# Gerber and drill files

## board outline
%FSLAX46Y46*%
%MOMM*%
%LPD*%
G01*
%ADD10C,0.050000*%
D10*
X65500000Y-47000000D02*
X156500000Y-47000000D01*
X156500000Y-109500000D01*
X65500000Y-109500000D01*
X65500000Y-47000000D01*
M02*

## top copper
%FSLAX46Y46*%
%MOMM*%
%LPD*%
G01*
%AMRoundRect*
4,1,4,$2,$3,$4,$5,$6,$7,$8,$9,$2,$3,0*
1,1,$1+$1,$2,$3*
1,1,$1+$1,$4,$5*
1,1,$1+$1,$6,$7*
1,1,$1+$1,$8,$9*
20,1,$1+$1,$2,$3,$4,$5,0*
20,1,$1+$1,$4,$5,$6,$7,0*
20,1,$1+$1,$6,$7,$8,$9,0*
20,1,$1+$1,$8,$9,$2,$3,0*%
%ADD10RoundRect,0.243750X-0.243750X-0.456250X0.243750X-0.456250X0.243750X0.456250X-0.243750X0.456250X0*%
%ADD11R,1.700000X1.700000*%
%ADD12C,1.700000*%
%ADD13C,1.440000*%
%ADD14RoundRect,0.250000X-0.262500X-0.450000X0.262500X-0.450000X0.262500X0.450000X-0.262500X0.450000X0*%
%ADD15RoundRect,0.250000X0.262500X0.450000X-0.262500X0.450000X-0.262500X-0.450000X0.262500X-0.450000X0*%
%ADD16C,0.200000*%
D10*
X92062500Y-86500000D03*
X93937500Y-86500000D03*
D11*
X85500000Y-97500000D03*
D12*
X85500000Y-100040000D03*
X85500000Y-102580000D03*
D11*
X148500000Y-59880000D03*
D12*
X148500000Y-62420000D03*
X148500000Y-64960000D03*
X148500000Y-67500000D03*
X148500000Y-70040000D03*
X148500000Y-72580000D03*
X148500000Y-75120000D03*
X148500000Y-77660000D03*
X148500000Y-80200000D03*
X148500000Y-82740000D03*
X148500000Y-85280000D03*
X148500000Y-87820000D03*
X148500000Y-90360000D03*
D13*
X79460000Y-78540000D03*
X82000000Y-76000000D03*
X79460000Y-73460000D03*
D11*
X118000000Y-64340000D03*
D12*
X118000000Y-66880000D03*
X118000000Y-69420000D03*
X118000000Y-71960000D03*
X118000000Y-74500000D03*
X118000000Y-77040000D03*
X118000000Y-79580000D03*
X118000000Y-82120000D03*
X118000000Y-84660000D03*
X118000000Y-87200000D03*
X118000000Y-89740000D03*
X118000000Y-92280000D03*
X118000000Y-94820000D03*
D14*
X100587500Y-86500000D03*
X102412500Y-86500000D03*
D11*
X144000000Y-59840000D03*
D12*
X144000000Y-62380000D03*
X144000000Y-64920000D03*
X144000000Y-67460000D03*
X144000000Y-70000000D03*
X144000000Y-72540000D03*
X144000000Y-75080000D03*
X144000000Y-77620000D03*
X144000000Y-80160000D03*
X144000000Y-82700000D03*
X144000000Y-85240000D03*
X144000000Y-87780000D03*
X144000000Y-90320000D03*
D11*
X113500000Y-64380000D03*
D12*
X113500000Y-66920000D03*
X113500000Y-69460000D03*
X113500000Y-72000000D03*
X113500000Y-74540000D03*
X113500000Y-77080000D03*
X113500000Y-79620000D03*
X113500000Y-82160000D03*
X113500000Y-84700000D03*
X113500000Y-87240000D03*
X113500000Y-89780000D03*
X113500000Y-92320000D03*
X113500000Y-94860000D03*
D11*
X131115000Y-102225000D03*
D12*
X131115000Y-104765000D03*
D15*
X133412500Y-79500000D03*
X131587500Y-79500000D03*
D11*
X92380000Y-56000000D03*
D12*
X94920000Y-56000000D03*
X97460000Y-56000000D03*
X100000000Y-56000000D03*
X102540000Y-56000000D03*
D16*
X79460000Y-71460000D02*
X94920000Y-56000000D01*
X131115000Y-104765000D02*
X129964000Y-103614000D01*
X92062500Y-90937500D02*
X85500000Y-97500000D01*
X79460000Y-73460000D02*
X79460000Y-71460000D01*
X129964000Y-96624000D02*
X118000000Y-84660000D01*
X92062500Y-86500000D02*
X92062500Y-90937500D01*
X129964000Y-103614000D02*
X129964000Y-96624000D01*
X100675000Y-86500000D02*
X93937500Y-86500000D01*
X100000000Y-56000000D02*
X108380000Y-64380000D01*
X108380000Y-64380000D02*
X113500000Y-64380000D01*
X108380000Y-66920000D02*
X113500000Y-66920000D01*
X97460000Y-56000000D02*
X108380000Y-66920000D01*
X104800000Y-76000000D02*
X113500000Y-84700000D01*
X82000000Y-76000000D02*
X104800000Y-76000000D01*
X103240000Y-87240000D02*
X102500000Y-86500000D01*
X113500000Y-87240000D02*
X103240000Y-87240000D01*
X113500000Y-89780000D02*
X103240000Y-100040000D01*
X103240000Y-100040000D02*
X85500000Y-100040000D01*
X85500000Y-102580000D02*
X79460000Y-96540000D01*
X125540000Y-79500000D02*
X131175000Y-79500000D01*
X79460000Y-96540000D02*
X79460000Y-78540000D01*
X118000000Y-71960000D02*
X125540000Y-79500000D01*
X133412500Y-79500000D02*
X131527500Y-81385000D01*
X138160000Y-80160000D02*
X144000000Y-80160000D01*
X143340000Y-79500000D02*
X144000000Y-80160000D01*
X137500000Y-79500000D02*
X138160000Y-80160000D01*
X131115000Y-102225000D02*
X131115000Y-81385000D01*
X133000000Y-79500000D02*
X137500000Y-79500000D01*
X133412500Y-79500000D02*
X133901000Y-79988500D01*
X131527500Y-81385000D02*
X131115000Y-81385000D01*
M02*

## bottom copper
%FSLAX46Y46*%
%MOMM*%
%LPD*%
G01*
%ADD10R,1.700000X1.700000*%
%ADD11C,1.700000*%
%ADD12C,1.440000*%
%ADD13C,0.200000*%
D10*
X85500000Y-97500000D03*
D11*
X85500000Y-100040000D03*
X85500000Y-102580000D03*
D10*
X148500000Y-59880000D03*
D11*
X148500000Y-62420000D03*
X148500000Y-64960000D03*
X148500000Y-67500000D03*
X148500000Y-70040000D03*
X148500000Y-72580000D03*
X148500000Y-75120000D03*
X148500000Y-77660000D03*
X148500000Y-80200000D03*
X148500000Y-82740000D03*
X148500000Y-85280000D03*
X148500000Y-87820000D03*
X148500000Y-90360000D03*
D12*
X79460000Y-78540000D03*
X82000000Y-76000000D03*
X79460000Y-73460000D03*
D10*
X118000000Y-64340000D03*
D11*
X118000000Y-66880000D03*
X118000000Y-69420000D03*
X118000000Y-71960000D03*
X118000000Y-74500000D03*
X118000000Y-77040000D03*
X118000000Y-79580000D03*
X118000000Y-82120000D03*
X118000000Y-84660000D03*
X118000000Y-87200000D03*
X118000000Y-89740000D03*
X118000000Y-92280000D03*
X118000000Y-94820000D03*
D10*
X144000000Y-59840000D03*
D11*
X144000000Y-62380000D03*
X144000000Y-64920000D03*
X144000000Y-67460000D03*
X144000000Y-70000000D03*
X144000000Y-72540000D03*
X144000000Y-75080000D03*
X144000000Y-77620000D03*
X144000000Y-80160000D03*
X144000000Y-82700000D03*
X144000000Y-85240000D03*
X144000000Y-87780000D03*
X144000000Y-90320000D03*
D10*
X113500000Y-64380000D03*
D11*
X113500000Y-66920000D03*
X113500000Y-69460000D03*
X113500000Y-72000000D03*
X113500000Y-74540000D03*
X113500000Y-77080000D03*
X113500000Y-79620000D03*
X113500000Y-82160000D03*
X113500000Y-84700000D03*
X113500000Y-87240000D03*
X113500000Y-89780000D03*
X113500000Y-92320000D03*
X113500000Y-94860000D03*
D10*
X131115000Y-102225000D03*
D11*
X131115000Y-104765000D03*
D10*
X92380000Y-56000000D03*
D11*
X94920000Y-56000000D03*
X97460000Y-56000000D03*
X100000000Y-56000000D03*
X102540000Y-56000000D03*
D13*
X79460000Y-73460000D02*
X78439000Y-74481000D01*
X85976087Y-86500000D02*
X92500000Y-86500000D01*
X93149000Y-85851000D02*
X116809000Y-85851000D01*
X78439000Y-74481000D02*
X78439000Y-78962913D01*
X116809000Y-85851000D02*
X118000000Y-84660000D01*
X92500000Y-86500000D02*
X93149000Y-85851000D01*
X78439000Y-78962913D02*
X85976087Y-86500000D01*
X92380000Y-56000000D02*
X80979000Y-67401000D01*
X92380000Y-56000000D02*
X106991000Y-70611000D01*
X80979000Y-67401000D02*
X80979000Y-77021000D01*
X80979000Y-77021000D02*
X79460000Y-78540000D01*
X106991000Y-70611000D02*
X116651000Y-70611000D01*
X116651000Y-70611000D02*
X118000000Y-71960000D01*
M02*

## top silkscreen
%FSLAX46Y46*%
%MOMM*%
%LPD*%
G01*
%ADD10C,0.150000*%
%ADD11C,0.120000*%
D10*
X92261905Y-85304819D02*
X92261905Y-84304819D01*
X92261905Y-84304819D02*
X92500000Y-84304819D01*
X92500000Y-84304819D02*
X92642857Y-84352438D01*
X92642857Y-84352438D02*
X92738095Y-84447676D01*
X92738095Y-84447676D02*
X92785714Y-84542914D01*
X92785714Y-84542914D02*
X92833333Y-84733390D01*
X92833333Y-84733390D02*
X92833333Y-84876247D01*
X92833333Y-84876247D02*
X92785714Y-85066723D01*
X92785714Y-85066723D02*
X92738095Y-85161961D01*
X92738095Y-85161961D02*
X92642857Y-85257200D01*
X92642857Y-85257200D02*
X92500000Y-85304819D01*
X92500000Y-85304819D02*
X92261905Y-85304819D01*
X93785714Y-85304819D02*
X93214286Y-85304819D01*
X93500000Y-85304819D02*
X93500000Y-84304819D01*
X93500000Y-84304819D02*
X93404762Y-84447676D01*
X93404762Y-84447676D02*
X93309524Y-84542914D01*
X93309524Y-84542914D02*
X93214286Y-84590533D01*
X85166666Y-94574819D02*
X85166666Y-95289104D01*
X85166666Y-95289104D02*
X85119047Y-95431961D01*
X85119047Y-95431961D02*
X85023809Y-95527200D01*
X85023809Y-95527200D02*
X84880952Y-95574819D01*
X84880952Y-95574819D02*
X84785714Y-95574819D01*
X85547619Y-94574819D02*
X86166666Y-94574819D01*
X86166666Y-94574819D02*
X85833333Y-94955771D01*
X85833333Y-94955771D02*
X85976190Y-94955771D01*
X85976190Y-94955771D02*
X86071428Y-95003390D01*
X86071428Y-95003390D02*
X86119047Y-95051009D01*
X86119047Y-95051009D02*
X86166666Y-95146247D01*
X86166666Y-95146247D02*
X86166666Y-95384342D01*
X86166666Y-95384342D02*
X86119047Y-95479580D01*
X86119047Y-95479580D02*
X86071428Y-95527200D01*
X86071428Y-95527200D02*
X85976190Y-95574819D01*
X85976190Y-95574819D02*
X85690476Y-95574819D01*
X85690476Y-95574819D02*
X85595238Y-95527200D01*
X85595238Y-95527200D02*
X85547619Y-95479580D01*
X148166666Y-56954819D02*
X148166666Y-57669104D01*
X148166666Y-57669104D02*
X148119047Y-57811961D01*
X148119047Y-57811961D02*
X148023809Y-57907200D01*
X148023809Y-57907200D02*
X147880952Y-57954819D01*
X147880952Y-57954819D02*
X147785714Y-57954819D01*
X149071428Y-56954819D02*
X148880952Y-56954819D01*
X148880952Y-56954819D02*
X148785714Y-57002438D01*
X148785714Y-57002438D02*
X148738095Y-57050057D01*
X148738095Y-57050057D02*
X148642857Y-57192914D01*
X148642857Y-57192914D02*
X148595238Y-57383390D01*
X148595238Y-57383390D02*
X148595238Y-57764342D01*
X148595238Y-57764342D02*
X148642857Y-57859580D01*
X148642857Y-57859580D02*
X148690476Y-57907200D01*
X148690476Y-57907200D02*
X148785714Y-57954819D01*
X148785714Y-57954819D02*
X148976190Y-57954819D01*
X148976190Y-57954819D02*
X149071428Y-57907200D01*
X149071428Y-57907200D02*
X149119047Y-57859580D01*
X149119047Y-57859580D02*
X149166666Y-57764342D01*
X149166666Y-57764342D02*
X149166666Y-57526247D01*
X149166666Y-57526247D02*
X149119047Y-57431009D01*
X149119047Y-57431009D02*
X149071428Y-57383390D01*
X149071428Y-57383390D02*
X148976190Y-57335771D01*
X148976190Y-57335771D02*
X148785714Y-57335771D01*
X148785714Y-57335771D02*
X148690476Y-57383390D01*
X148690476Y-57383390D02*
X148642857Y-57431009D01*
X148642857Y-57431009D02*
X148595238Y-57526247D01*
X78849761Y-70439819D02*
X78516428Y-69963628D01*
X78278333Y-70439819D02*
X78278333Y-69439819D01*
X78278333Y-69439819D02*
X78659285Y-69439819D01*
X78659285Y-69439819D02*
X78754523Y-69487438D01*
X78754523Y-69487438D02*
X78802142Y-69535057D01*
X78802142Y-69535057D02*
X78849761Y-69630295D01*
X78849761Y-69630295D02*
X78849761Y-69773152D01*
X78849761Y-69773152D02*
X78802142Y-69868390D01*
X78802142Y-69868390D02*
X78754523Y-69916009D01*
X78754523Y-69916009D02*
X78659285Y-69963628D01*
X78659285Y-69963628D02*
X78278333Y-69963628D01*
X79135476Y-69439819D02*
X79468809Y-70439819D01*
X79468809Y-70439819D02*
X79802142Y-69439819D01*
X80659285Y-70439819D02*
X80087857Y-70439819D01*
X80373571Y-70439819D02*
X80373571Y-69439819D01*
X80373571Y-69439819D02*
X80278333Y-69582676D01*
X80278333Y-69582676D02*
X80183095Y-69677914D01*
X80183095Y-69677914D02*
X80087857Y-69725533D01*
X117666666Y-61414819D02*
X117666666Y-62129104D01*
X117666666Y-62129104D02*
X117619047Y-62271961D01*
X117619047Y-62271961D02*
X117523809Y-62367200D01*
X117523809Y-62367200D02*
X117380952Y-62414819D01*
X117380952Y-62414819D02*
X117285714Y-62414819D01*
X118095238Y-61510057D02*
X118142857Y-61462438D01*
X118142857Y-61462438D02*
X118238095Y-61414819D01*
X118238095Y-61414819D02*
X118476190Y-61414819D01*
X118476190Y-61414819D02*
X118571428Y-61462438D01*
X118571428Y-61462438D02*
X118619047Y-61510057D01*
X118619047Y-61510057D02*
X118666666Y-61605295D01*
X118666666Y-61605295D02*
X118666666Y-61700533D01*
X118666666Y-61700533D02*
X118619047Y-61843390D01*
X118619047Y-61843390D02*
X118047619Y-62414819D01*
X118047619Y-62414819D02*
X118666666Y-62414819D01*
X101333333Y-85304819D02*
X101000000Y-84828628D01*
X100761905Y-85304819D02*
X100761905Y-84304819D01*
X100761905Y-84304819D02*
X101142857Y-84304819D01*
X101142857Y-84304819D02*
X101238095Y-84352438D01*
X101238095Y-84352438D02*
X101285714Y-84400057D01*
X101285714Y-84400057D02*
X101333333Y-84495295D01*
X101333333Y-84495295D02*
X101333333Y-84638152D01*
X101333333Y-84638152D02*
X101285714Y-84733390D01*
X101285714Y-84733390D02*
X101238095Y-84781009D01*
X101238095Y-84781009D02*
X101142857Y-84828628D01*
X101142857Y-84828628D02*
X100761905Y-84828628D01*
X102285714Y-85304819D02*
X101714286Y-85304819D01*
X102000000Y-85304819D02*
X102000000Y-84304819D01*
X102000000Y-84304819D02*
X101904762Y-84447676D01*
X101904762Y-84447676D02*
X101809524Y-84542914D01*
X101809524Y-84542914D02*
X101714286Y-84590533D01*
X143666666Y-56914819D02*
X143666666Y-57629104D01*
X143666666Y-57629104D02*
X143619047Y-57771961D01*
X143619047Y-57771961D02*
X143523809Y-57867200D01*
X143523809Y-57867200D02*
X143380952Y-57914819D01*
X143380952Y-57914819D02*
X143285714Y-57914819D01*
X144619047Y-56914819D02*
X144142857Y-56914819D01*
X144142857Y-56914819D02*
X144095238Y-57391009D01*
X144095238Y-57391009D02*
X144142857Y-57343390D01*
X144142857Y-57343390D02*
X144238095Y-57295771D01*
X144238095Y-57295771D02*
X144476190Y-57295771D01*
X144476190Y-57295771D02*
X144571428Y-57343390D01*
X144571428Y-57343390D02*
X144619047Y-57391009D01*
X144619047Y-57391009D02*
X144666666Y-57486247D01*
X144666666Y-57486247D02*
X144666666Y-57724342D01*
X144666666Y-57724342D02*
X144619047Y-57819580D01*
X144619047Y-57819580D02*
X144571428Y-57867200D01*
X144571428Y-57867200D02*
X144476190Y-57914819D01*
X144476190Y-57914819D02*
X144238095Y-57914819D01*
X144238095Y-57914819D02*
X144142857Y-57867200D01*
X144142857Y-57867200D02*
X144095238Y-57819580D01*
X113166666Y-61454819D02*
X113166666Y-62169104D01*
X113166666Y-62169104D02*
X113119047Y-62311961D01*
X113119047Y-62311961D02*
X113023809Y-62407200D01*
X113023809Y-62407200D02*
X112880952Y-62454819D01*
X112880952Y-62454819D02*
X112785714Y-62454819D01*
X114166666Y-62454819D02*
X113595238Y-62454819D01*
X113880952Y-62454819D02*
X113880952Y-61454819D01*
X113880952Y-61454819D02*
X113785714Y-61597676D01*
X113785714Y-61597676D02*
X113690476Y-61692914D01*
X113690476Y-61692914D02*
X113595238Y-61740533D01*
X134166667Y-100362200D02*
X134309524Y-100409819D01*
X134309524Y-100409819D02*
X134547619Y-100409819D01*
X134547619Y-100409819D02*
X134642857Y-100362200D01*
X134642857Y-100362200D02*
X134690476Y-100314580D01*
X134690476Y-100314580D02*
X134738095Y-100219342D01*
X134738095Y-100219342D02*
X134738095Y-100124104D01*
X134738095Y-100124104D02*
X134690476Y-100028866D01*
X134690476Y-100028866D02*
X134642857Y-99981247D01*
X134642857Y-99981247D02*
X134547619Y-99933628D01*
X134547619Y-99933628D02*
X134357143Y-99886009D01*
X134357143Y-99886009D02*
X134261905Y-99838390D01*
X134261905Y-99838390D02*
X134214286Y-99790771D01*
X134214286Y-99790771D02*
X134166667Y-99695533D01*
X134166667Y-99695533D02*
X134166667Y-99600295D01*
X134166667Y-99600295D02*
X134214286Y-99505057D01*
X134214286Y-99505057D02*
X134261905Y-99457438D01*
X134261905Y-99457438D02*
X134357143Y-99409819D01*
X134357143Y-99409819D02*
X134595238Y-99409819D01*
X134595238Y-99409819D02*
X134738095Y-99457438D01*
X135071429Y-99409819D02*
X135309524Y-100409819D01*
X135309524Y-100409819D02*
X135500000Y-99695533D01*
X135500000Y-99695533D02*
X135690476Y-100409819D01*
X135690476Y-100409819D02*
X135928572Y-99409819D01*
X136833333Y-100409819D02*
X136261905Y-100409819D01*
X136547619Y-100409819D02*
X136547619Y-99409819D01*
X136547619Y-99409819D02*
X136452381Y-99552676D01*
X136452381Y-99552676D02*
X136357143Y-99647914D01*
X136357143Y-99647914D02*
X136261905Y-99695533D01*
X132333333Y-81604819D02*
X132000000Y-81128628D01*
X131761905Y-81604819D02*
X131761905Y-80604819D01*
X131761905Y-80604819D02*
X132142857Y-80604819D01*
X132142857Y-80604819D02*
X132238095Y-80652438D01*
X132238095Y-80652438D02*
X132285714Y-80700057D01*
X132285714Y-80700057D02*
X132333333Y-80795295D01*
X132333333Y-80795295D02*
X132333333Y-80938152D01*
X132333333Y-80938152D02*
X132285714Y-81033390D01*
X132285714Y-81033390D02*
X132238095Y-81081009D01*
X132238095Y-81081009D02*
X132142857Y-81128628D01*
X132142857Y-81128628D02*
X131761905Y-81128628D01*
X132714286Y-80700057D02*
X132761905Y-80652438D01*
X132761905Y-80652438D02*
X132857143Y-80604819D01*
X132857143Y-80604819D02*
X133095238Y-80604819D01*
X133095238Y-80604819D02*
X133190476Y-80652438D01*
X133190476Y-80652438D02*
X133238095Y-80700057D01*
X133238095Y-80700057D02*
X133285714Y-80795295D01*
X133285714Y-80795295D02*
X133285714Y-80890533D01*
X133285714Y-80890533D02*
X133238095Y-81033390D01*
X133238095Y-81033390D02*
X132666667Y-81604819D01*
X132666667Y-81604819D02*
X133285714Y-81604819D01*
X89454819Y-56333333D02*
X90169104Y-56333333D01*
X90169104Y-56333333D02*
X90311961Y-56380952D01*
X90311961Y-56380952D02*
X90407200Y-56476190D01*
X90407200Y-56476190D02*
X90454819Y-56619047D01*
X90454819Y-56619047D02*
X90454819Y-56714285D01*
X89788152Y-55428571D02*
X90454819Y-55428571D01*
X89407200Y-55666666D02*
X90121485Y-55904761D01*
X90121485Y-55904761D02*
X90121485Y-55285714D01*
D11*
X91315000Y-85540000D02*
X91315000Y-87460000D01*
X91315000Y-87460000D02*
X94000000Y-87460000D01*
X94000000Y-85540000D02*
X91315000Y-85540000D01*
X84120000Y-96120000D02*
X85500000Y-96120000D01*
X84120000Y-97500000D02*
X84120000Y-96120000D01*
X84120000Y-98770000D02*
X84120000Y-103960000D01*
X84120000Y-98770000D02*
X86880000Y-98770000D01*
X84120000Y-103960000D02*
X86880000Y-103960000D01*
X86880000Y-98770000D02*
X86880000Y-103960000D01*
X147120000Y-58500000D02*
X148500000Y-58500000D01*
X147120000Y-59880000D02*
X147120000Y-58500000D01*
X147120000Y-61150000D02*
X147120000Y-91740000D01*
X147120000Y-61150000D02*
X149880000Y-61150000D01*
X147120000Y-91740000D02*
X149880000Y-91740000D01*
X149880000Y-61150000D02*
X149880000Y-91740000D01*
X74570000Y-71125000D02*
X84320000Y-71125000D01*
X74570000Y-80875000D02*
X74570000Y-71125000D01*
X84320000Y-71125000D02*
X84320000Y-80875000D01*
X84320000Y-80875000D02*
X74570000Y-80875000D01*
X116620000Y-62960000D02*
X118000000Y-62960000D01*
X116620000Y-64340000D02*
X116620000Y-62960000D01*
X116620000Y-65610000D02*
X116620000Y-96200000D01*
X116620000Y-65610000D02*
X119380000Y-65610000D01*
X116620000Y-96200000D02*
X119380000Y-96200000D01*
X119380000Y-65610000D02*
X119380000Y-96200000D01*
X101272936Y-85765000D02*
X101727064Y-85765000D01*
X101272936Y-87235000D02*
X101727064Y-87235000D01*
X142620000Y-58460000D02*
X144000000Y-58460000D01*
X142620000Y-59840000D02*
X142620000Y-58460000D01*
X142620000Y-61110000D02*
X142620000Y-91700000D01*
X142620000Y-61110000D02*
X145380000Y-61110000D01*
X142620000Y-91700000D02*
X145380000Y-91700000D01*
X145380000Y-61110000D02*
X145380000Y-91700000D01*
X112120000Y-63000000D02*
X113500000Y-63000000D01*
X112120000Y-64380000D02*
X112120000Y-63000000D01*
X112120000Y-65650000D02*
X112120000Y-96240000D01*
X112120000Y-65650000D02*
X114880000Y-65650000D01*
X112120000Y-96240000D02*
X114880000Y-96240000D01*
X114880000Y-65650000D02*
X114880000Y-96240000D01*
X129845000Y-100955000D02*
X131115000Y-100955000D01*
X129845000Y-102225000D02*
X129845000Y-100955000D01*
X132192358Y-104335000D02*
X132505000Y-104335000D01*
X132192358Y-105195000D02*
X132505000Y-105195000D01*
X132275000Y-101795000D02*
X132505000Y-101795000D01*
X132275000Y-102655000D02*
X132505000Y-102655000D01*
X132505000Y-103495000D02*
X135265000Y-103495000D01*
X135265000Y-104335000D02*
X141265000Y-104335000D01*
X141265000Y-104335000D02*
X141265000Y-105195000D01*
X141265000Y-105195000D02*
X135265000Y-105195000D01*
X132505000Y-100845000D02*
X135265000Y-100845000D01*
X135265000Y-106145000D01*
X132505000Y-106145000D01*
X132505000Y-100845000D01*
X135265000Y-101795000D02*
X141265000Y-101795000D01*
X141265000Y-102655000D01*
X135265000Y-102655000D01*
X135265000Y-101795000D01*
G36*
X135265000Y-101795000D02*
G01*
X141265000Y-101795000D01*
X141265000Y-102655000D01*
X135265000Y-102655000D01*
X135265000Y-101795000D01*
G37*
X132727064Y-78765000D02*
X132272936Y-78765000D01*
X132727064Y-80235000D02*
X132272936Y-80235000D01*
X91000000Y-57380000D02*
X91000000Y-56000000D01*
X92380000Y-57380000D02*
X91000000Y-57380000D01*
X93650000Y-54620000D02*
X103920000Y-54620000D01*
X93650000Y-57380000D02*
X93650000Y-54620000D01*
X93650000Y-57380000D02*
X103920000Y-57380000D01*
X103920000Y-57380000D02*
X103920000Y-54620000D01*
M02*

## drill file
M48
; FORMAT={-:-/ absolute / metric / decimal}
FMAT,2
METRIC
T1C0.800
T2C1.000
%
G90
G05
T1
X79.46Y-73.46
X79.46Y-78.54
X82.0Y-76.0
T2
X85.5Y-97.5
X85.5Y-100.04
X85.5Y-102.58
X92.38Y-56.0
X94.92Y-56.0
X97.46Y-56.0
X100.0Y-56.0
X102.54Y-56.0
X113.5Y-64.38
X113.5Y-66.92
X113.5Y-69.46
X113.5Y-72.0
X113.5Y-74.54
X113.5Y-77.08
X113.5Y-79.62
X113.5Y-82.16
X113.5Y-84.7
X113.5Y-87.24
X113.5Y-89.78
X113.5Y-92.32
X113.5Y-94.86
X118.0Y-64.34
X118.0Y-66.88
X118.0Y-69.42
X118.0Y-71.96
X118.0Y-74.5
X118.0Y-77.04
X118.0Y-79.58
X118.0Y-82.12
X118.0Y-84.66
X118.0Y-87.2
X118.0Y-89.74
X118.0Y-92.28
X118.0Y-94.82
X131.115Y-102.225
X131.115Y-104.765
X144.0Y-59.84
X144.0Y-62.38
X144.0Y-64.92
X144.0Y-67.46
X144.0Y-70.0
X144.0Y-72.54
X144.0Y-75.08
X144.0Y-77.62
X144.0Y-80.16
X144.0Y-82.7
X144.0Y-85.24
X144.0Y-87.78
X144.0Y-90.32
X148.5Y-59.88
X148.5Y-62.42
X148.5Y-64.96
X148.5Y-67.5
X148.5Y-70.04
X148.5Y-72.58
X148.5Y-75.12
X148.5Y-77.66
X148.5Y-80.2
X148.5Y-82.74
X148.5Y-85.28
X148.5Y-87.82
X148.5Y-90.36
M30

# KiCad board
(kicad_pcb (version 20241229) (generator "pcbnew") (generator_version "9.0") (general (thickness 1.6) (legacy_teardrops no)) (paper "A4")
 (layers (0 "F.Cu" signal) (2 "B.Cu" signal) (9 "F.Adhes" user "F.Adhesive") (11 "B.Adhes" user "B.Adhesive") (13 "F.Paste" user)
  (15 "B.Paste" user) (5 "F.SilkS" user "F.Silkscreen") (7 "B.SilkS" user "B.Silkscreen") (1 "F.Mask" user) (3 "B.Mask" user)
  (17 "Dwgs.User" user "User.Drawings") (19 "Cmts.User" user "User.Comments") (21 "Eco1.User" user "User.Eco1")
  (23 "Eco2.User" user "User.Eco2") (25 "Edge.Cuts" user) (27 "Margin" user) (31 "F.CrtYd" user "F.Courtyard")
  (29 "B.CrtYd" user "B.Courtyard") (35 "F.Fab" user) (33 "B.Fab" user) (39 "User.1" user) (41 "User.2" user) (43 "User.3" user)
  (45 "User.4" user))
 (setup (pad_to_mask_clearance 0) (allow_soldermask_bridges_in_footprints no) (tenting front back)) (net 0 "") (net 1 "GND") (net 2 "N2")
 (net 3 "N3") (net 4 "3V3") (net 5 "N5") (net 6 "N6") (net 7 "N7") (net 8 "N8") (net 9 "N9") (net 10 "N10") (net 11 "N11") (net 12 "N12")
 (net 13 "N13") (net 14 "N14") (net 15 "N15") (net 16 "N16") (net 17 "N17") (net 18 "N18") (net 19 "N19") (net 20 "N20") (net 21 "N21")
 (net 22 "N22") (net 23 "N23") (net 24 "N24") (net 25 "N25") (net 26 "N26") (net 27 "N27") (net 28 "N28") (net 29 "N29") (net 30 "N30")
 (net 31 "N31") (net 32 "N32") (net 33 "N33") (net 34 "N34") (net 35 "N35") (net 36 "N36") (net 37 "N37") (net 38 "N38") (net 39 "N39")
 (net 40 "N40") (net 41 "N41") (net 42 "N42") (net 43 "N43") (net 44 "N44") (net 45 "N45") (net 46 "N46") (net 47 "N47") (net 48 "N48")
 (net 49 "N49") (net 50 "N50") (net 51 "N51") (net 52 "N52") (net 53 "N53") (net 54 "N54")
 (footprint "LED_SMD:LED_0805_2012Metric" (layer "F.Cu") (at 93 86.5)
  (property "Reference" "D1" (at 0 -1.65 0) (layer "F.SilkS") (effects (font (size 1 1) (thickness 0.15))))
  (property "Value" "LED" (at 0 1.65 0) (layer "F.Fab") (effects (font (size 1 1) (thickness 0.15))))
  (fp_line (start -1.685 -0.96) (end -1.685 0.96) (stroke (width 0.12) (type solid)) (layer "F.SilkS"))
  (fp_line (start -1.685 0.96) (end 1 0.96) (stroke (width 0.12) (type solid)) (layer "F.SilkS"))
  (fp_line (start 1 -0.96) (end -1.685 -0.96) (stroke (width 0.12) (type solid)) (layer "F.SilkS"))
  (pad "1" smd roundrect (at -0.9375 0) (size 0.975 1.4) (layers "F.Cu" "F.Mask" "F.Paste") (roundrect_rratio 0.25) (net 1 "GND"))
  (pad "2" smd roundrect (at 0.9375 0) (size 0.975 1.4) (layers "F.Cu" "F.Mask" "F.Paste") (roundrect_rratio 0.25) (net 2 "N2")))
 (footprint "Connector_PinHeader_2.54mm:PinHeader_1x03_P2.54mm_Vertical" (layer "F.Cu") (at 85.5 97.5)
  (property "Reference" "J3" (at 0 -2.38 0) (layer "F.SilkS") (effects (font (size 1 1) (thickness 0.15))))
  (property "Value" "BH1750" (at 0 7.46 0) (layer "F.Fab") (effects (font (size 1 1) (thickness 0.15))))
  (fp_line (start -1.38 -1.38) (end 0 -1.38) (stroke (width 0.12) (type solid)) (layer "F.SilkS"))
  (fp_line (start -1.38 0) (end -1.38 -1.38) (stroke (width 0.12) (type solid)) (layer "F.SilkS"))
  (fp_line (start -1.38 1.27) (end -1.38 6.46) (stroke (width 0.12) (type solid)) (layer "F.SilkS"))
  (fp_line (start -1.38 1.27) (end 1.38 1.27) (stroke (width 0.12) (type solid)) (layer "F.SilkS"))
  (fp_line (start -1.38 6.46) (end 1.38 6.46) (stroke (width 0.12) (type solid)) (layer "F.SilkS"))
  (fp_line (start 1.38 1.27) (end 1.38 6.46) (stroke (width 0.12) (type solid)) (layer "F.SilkS"))
  (pad "1" thru_hole rect (at 0 0) (size 1.7 1.7) (drill 1) (layers "*.Cu" "*.Mask") (remove_unused_layers no) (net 1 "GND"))
  (pad "2" thru_hole circle (at 0 2.54) (size 1.7 1.7) (drill 1) (layers "*.Cu" "*.Mask") (remove_unused_layers no) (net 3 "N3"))
  (pad "3" thru_hole circle (at 0 5.08) (size 1.7 1.7) (drill 1) (layers "*.Cu" "*.Mask") (remove_unused_layers no) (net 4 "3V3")))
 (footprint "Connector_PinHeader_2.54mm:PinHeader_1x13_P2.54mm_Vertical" (layer "F.Cu") (at 148.5 59.88)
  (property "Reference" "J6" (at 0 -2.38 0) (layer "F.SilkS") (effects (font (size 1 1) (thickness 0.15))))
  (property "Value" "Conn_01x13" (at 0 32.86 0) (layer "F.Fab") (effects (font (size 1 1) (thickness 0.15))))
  (fp_line (start -1.38 -1.38) (end 0 -1.38) (stroke (width 0.12) (type solid)) (layer "F.SilkS"))
  (fp_line (start -1.38 0) (end -1.38 -1.38) (stroke (width 0.12) (type solid)) (layer "F.SilkS"))
  (fp_line (start -1.38 1.27) (end -1.38 31.86) (stroke (width 0.12) (type solid)) (layer "F.SilkS"))
  (fp_line (start -1.38 1.27) (end 1.38 1.27) (stroke (width 0.12) (type solid)) (layer "F.SilkS"))
  (fp_line (start -1.38 31.86) (end 1.38 31.86) (stroke (width 0.12) (type solid)) (layer "F.SilkS"))
  (fp_line (start 1.38 1.27) (end 1.38 31.86) (stroke (width 0.12) (type solid)) (layer "F.SilkS"))
  (pad "1" thru_hole rect (at 0 0) (size 1.7 1.7) (drill 1) (layers "*.Cu" "*.Mask") (remove_unused_layers no) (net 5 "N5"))
  (pad "2" thru_hole circle (at 0 2.54) (size 1.7 1.7) (drill 1) (layers "*.Cu" "*.Mask") (remove_unused_layers no) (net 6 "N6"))
  (pad "3" thru_hole circle (at 0 5.08) (size 1.7 1.7) (drill 1) (layers "*.Cu" "*.Mask") (remove_unused_layers no) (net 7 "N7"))
  (pad "4" thru_hole circle (at 0 7.62) (size 1.7 1.7) (drill 1) (layers "*.Cu" "*.Mask") (remove_unused_layers no) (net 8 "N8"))
  (pad "5" thru_hole circle (at 0 10.16) (size 1.7 1.7) (drill 1) (layers "*.Cu" "*.Mask") (remove_unused_layers no) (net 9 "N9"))
  (pad "6" thru_hole circle (at 0 12.7) (size 1.7 1.7) (drill 1) (layers "*.Cu" "*.Mask") (remove_unused_layers no) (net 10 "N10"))
  (pad "7" thru_hole circle (at 0 15.24) (size 1.7 1.7) (drill 1) (layers "*.Cu" "*.Mask") (remove_unused_layers no) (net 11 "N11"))
  (pad "8" thru_hole circle (at 0 17.78) (size 1.7 1.7) (drill 1) (layers "*.Cu" "*.Mask") (remove_unused_layers no) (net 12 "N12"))
  (pad "9" thru_hole circle (at 0 20.32) (size 1.7 1.7) (drill 1) (layers "*.Cu" "*.Mask") (remove_unused_layers no) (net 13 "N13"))
  (pad "10" thru_hole circle (at 0 22.86) (size 1.7 1.7) (drill 1) (layers "*.Cu" "*.Mask") (remove_unused_layers no) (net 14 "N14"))
  (pad "11" thru_hole circle (at 0 25.4) (size 1.7 1.7) (drill 1) (layers "*.Cu" "*.Mask") (remove_unused_layers no) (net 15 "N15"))
  (pad "12" thru_hole circle (at 0 27.94) (size 1.7 1.7) (drill 1) (layers "*.Cu" "*.Mask") (remove_unused_layers no) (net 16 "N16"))
  (pad "13" thru_hole circle (at 0 30.48) (size 1.7 1.7) (drill 1) (layers "*.Cu" "*.Mask") (remove_unused_layers no) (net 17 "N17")))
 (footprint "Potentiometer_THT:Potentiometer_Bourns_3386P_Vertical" (layer "F.Cu") (at 79.46 78.54)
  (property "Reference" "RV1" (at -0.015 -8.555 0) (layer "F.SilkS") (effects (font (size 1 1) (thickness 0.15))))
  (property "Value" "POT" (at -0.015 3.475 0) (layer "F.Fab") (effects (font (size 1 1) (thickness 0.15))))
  (fp_line (start -4.89 -7.415) (end 4.86 -7.415) (stroke (width 0.12) (type solid)) (layer "F.SilkS"))
  (fp_line (start -4.89 2.335) (end -4.89 -7.415) (stroke (width 0.12) (type solid)) (layer "F.SilkS"))
  (fp_line (start 4.86 -7.415) (end 4.86 2.335) (stroke (width 0.12) (type solid)) (layer "F.SilkS"))
  (fp_line (start 4.86 2.335) (end -4.89 2.335) (stroke (width 0.12) (type solid)) (layer "F.SilkS"))
  (pad "1" thru_hole circle (at 0 0) (size 1.44 1.44) (drill 0.8) (layers "*.Cu" "*.Mask") (remove_unused_layers no) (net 4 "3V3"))
  (pad "2" thru_hole circle (at 2.54 -2.54) (size 1.44 1.44) (drill 0.8) (layers "*.Cu" "*.Mask") (remove_unused_layers no) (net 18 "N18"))
  (pad "3" thru_hole circle (at 0 -5.08) (size 1.44 1.44) (drill 0.8) (layers "*.Cu" "*.Mask") (remove_unused_layers no) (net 1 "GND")))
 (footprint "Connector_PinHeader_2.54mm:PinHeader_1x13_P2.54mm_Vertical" (layer "F.Cu") (at 118 64.34)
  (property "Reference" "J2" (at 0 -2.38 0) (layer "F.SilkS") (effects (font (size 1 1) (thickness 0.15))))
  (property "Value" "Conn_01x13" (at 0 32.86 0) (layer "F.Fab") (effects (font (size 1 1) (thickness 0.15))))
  (fp_line (start -1.38 -1.38) (end 0 -1.38) (stroke (width 0.12) (type solid)) (layer "F.SilkS"))
  (fp_line (start -1.38 0) (end -1.38 -1.38) (stroke (width 0.12) (type solid)) (layer "F.SilkS"))
  (fp_line (start -1.38 1.27) (end -1.38 31.86) (stroke (width 0.12) (type solid)) (layer "F.SilkS"))
  (fp_line (start -1.38 1.27) (end 1.38 1.27) (stroke (width 0.12) (type solid)) (layer "F.SilkS"))
  (fp_line (start -1.38 31.86) (end 1.38 31.86) (stroke (width 0.12) (type solid)) (layer "F.SilkS"))
  (fp_line (start 1.38 1.27) (end 1.38 31.86) (stroke (width 0.12) (type solid)) (layer "F.SilkS"))
  (pad "1" thru_hole rect (at 0 0) (size 1.7 1.7) (drill 1) (layers "*.Cu" "*.Mask") (remove_unused_layers no) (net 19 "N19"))
  (pad "2" thru_hole circle (at 0 2.54) (size 1.7 1.7) (drill 1) (layers "*.Cu" "*.Mask") (remove_unused_layers no) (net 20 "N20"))
  (pad "3" thru_hole circle (at 0 5.08) (size 1.7 1.7) (drill 1) (layers "*.Cu" "*.Mask") (remove_unused_layers no) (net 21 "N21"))
  (pad "4" thru_hole circle (at 0 7.62) (size 1.7 1.7) (drill 1) (layers "*.Cu" "*.Mask") (remove_unused_layers no) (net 4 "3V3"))
  (pad "5" thru_hole circle (at 0 10.16) (size 1.7 1.7) (drill 1) (layers "*.Cu" "*.Mask") (remove_unused_layers no) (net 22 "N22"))
  (pad "6" thru_hole circle (at 0 12.7) (size 1.7 1.7) (drill 1) (layers "*.Cu" "*.Mask") (remove_unused_layers no) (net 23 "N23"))
  (pad "7" thru_hole circle (at 0 15.24) (size 1.7 1.7) (drill 1) (layers "*.Cu" "*.Mask") (remove_unused_layers no) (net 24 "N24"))
  (pad "8" thru_hole circle (at 0 17.78) (size 1.7 1.7) (drill 1) (layers "*.Cu" "*.Mask") (remove_unused_layers no) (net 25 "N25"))
  (pad "9" thru_hole circle (at 0 20.32) (size 1.7 1.7) (drill 1) (layers "*.Cu" "*.Mask") (remove_unused_layers no) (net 1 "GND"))
  (pad "10" thru_hole circle (at 0 22.86) (size 1.7 1.7) (drill 1) (layers "*.Cu" "*.Mask") (remove_unused_layers no) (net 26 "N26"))
  (pad "11" thru_hole circle (at 0 25.4) (size 1.7 1.7) (drill 1) (layers "*.Cu" "*.Mask") (remove_unused_layers no) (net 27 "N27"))
  (pad "12" thru_hole circle (at 0 27.94) (size 1.7 1.7) (drill 1) (layers "*.Cu" "*.Mask") (remove_unused_layers no) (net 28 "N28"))
  (pad "13" thru_hole circle (at 0 30.48) (size 1.7 1.7) (drill 1) (layers "*.Cu" "*.Mask") (remove_unused_layers no) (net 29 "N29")))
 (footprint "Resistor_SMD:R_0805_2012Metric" (layer "F.Cu") (at 101.5 86.5)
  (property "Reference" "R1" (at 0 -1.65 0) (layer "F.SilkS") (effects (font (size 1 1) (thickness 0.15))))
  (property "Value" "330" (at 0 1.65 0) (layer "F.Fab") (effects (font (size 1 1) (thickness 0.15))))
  (fp_line (start -0.227064 -0.735) (end 0.227064 -0.735) (stroke (width 0.12) (type solid)) (layer "F.SilkS"))
  (fp_line (start -0.227064 0.735) (end 0.227064 0.735) (stroke (width 0.12) (type solid)) (layer "F.SilkS"))
  (pad "1" smd roundrect (at -0.9125 0) (size 1.025 1.4) (layers "F.Cu" "F.Mask" "F.Paste") (roundrect_rratio 0.243902) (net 2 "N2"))
  (pad "2" smd roundrect (at 0.9125 0) (size 1.025 1.4) (layers "F.Cu" "F.Mask" "F.Paste") (roundrect_rratio 0.243902) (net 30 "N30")))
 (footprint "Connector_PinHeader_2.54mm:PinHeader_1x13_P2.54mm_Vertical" (layer "F.Cu") (at 144 59.84)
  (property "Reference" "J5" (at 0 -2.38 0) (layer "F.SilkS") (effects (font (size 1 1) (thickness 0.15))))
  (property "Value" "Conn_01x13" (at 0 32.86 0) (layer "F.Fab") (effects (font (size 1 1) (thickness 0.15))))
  (fp_line (start -1.38 -1.38) (end 0 -1.38) (stroke (width 0.12) (type solid)) (layer "F.SilkS"))
  (fp_line (start -1.38 0) (end -1.38 -1.38) (stroke (width 0.12) (type solid)) (layer "F.SilkS"))
  (fp_line (start -1.38 1.27) (end -1.38 31.86) (stroke (width 0.12) (type solid)) (layer "F.SilkS"))
  (fp_line (start -1.38 1.27) (end 1.38 1.27) (stroke (width 0.12) (type solid)) (layer "F.SilkS"))
  (fp_line (start -1.38 31.86) (end 1.38 31.86) (stroke (width 0.12) (type solid)) (layer "F.SilkS"))
  (fp_line (start 1.38 1.27) (end 1.38 31.86) (stroke (width 0.12) (type solid)) (layer "F.SilkS"))
  (pad "1" thru_hole rect (at 0 0) (size 1.7 1.7) (drill 1) (layers "*.Cu" "*.Mask") (remove_unused_layers no) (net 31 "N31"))
  (pad "2" thru_hole circle (at 0 2.54) (size 1.7 1.7) (drill 1) (layers "*.Cu" "*.Mask") (remove_unused_layers no) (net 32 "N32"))
  (pad "3" thru_hole circle (at 0 5.08) (size 1.7 1.7) (drill 1) (layers "*.Cu" "*.Mask") (remove_unused_layers no) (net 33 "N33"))
  (pad "4" thru_hole circle (at 0 7.62) (size 1.7 1.7) (drill 1) (layers "*.Cu" "*.Mask") (remove_unused_layers no) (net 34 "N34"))
  (pad "5" thru_hole circle (at 0 10.16) (size 1.7 1.7) (drill 1) (layers "*.Cu" "*.Mask") (remove_unused_layers no) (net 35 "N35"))
  (pad "6" thru_hole circle (at 0 12.7) (size 1.7 1.7) (drill 1) (layers "*.Cu" "*.Mask") (remove_unused_layers no) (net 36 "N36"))
  (pad "7" thru_hole circle (at 0 15.24) (size 1.7 1.7) (drill 1) (layers "*.Cu" "*.Mask") (remove_unused_layers no) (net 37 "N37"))
  (pad "8" thru_hole circle (at 0 17.78) (size 1.7 1.7) (drill 1) (layers "*.Cu" "*.Mask") (remove_unused_layers no) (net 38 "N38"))
  (pad "9" thru_hole circle (at 0 20.32) (size 1.7 1.7) (drill 1) (layers "*.Cu" "*.Mask") (remove_unused_layers no) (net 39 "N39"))
  (pad "10" thru_hole circle (at 0 22.86) (size 1.7 1.7) (drill 1) (layers "*.Cu" "*.Mask") (remove_unused_layers no) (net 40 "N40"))
  (pad "11" thru_hole circle (at 0 25.4) (size 1.7 1.7) (drill 1) (layers "*.Cu" "*.Mask") (remove_unused_layers no) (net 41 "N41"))
  (pad "12" thru_hole circle (at 0 27.94) (size 1.7 1.7) (drill 1) (layers "*.Cu" "*.Mask") (remove_unused_layers no) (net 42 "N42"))
  (pad "13" thru_hole circle (at 0 30.48) (size 1.7 1.7) (drill 1) (layers "*.Cu" "*.Mask") (remove_unused_layers no) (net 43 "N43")))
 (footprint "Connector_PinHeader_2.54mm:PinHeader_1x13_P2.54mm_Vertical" (layer "F.Cu") (at 113.5 64.38)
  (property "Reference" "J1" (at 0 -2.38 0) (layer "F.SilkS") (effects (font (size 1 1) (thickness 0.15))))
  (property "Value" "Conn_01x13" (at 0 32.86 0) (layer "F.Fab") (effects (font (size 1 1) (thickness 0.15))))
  (fp_line (start -1.38 -1.38) (end 0 -1.38) (stroke (width 0.12) (type solid)) (layer "F.SilkS"))
  (fp_line (start -1.38 0) (end -1.38 -1.38) (stroke (width 0.12) (type solid)) (layer "F.SilkS"))
  (fp_line (start -1.38 1.27) (end -1.38 31.86) (stroke (width 0.12) (type solid)) (layer "F.SilkS"))
  (fp_line (start -1.38 1.27) (end 1.38 1.27) (stroke (width 0.12) (type solid)) (layer "F.SilkS"))
  (fp_line (start -1.38 31.86) (end 1.38 31.86) (stroke (width 0.12) (type solid)) (layer "F.SilkS"))
  (fp_line (start 1.38 1.27) (end 1.38 31.86) (stroke (width 0.12) (type solid)) (layer "F.SilkS"))
  (pad "1" thru_hole rect (at 0 0) (size 1.7 1.7) (drill 1) (layers "*.Cu" "*.Mask") (remove_unused_layers no) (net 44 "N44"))
  (pad "2" thru_hole circle (at 0 2.54) (size 1.7 1.7) (drill 1) (layers "*.Cu" "*.Mask") (remove_unused_layers no) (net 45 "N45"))
  (pad "3" thru_hole circle (at 0 5.08) (size 1.7 1.7) (drill 1) (layers "*.Cu" "*.Mask") (remove_unused_layers no) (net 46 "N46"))
  (pad "4" thru_hole circle (at 0 7.62) (size 1.7 1.7) (drill 1) (layers "*.Cu" "*.Mask") (remove_unused_layers no) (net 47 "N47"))
  (pad "5" thru_hole circle (at 0 10.16) (size 1.7 1.7) (drill 1) (layers "*.Cu" "*.Mask") (remove_unused_layers no) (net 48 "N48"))
  (pad "6" thru_hole circle (at 0 12.7) (size 1.7 1.7) (drill 1) (layers "*.Cu" "*.Mask") (remove_unused_layers no) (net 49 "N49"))
  (pad "7" thru_hole circle (at 0 15.24) (size 1.7 1.7) (drill 1) (layers "*.Cu" "*.Mask") (remove_unused_layers no) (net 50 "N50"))
  (pad "8" thru_hole circle (at 0 17.78) (size 1.7 1.7) (drill 1) (layers "*.Cu" "*.Mask") (remove_unused_layers no) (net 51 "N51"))
  (pad "9" thru_hole circle (at 0 20.32) (size 1.7 1.7) (drill 1) (layers "*.Cu" "*.Mask") (remove_unused_layers no) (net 18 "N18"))
  (pad "10" thru_hole circle (at 0 22.86) (size 1.7 1.7) (drill 1) (layers "*.Cu" "*.Mask") (remove_unused_layers no) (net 30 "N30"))
  (pad "11" thru_hole circle (at 0 25.4) (size 1.7 1.7) (drill 1) (layers "*.Cu" "*.Mask") (remove_unused_layers no) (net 3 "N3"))
  (pad "12" thru_hole circle (at 0 27.94) (size 1.7 1.7) (drill 1) (layers "*.Cu" "*.Mask") (remove_unused_layers no) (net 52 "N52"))
  (pad "13" thru_hole circle (at 0 30.48) (size 1.7 1.7) (drill 1) (layers "*.Cu" "*.Mask") (remove_unused_layers no) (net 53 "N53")))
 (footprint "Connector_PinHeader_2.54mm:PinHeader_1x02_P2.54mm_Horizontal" (layer "F.Cu") (at 131.115 102.225)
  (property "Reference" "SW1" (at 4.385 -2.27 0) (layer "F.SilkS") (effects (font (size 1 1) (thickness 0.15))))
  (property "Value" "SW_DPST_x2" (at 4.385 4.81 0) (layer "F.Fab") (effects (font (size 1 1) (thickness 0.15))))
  (fp_line (start -1.27 -1.27) (end 0 -1.27) (stroke (width 0.12) (type solid)) (layer "F.SilkS"))
  (fp_line (start -1.27 0) (end -1.27 -1.27) (stroke (width 0.12) (type solid)) (layer "F.SilkS"))
  (fp_line (start 1.077358 2.11) (end 1.39 2.11) (stroke (width 0.12) (type solid)) (layer "F.SilkS"))
  (fp_line (start 1.077358 2.97) (end 1.39 2.97) (stroke (width 0.12) (type solid)) (layer "F.SilkS"))
  (fp_line (start 1.16 -0.43) (end 1.39 -0.43) (stroke (width 0.12) (type solid)) (layer "F.SilkS"))
  (fp_line (start 1.16 0.43) (end 1.39 0.43) (stroke (width 0.12) (type solid)) (layer "F.SilkS"))
  (fp_line (start 1.39 1.27) (end 4.15 1.27) (stroke (width 0.12) (type solid)) (layer "F.SilkS"))
  (fp_line (start 4.15 2.11) (end 10.15 2.11) (stroke (width 0.12) (type solid)) (layer "F.SilkS"))
  (fp_line (start 10.15 2.11) (end 10.15 2.97) (stroke (width 0.12) (type solid)) (layer "F.SilkS"))
  (fp_line (start 10.15 2.97) (end 4.15 2.97) (stroke (width 0.12) (type solid)) (layer "F.SilkS"))
  (fp_rect (start 1.39 -1.38) (end 4.15 3.92) (stroke (width 0.12) (type solid)) (fill no) (layer "F.SilkS"))
  (fp_rect (start 4.15 -0.43) (end 10.15 0.43) (stroke (width 0.12) (type solid)) (fill yes) (layer "F.SilkS"))
  (pad "1" thru_hole rect (at 0 0) (size 1.7 1.7) (drill 1) (layers "*.Cu" "*.Mask") (remove_unused_layers no) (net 39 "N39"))
  (pad "2" thru_hole circle (at 0 2.54) (size 1.7 1.7) (drill 1) (layers "*.Cu" "*.Mask") (remove_unused_layers no) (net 1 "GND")))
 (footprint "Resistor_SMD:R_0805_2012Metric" (layer "F.Cu") (at 132.5 79.5 180)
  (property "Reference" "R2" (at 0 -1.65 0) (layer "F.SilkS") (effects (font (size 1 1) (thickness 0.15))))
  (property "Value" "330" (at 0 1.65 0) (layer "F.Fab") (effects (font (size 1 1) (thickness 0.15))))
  (fp_line (start -0.227064 0.735) (end 0.227064 0.735) (stroke (width 0.12) (type solid)) (layer "F.SilkS"))
  (fp_line (start -0.227064 -0.735) (end 0.227064 -0.735) (stroke (width 0.12) (type solid)) (layer "F.SilkS"))
  (pad "1" smd roundrect (at -0.9125 0 180) (size 1.025 1.4) (layers "F.Cu" "F.Mask" "F.Paste") (roundrect_rratio 0.243902) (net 39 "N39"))
  (pad "2" smd roundrect (at 0.9125 0 180) (size 1.025 1.4) (layers "F.Cu" "F.Mask" "F.Paste") (roundrect_rratio 0.243902) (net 4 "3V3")))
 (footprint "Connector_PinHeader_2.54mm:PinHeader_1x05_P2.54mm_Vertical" (layer "F.Cu") (at 92.38 56 90)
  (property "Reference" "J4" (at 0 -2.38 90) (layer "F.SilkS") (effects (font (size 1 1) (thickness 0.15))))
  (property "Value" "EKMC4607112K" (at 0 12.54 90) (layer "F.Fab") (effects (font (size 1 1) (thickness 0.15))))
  (fp_line (start -1.38 -1.38) (end 0 -1.38) (stroke (width 0.12) (type solid)) (layer "F.SilkS"))
  (fp_line (start -1.38 0) (end -1.38 -1.38) (stroke (width 0.12) (type solid)) (layer "F.SilkS"))
  (fp_line (start 1.38 1.27) (end 1.38 11.54) (stroke (width 0.12) (type solid)) (layer "F.SilkS"))
  (fp_line (start -1.38 1.27) (end 1.38 1.27) (stroke (width 0.12) (type solid)) (layer "F.SilkS"))
  (fp_line (start -1.38 1.27) (end -1.38 11.54) (stroke (width 0.12) (type solid)) (layer "F.SilkS"))
  (fp_line (start -1.38 11.54) (end 1.38 11.54) (stroke (width 0.12) (type solid)) (layer "F.SilkS"))
  (pad "1" thru_hole rect (at 0 0 90) (size 1.7 1.7) (drill 1) (layers "*.Cu" "*.Mask") (remove_unused_layers no) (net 4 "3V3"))
  (pad "2" thru_hole circle (at 0 2.54 90) (size 1.7 1.7) (drill 1) (layers "*.Cu" "*.Mask") (remove_unused_layers no) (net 1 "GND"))
  (pad "3" thru_hole circle (at 0 5.08 90) (size 1.7 1.7) (drill 1) (layers "*.Cu" "*.Mask") (remove_unused_layers no) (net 45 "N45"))
  (pad "4" thru_hole circle (at 0 7.62 90) (size 1.7 1.7) (drill 1) (layers "*.Cu" "*.Mask") (remove_unused_layers no) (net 44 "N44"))
  (pad "5" thru_hole circle (at 0 10.16 90) (size 1.7 1.7) (drill 1) (layers "*.Cu" "*.Mask") (remove_unused_layers no) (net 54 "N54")))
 (gr_rect (start 65.5 47) (end 156.5 109.5) (stroke (width 0.05) (type default)) (fill no) (layer "Edge.Cuts"))
 (segment (start 79.46 71.46) (end 94.92 56) (width 0.2) (layer "F.Cu") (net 1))
 (segment (start 131.115 104.765) (end 129.964 103.614) (width 0.2) (layer "F.Cu") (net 1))
 (segment (start 92.0625 90.9375) (end 85.5 97.5) (width 0.2) (layer "F.Cu") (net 1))
 (segment (start 79.46 73.46) (end 79.46 71.46) (width 0.2) (layer "F.Cu") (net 1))
 (segment (start 129.964 96.624) (end 118 84.66) (width 0.2) (layer "F.Cu") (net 1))
 (segment (start 92.0625 86.5) (end 92.0625 90.9375) (width 0.2) (layer "F.Cu") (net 1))
 (segment (start 129.964 103.614) (end 129.964 96.624) (width 0.2) (layer "F.Cu") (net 1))
 (segment (start 79.46 73.46) (end 78.439 74.481) (width 0.2) (layer "B.Cu") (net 1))
 (segment (start 85.976087 86.5) (end 92.5 86.5) (width 0.2) (layer "B.Cu") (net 1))
 (segment (start 93.149 85.851) (end 116.809 85.851) (width 0.2) (layer "B.Cu") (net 1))
 (segment (start 78.439 74.481) (end 78.439 78.962913) (width 0.2) (layer "B.Cu") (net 1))
 (segment (start 116.809 85.851) (end 118 84.66) (width 0.2) (layer "B.Cu") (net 1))
 (segment (start 92.5 86.5) (end 93.149 85.851) (width 0.2) (layer "B.Cu") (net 1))
 (segment (start 78.439 78.962913) (end 85.976087 86.5) (width 0.2) (layer "B.Cu") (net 1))
 (segment (start 100.675 86.5) (end 93.9375 86.5) (width 0.2) (layer "F.Cu") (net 2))
 (segment (start 100 56) (end 108.38 64.38) (width 0.2) (layer "F.Cu") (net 44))
 (segment (start 108.38 64.38) (end 113.5 64.38) (width 0.2) (layer "F.Cu") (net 44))
 (segment (start 108.38 66.92) (end 113.5 66.92) (width 0.2) (layer "F.Cu") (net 45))
 (segment (start 97.46 56) (end 108.38 66.92) (width 0.2) (layer "F.Cu") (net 45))
 (segment (start 104.8 76) (end 113.5 84.7) (width 0.2) (layer "F.Cu") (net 18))
 (segment (start 82 76) (end 104.8 76) (width 0.2) (layer "F.Cu") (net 18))
 (segment (start 103.24 87.24) (end 102.5 86.5) (width 0.2) (layer "F.Cu") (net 30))
 (segment (start 113.5 87.24) (end 103.24 87.24) (width 0.2) (layer "F.Cu") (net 30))
 (segment (start 113.5 89.78) (end 103.24 100.04) (width 0.2) (layer "F.Cu") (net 3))
 (segment (start 103.24 100.04) (end 85.5 100.04) (width 0.2) (layer "F.Cu") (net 3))
 (segment (start 85.5 102.58) (end 79.46 96.54) (width 0.2) (layer "F.Cu") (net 4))
 (segment (start 125.54 79.5) (end 131.175 79.5) (width 0.2) (layer "F.Cu") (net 4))
 (segment (start 79.46 96.54) (end 79.46 78.54) (width 0.2) (layer "F.Cu") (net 4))
 (segment (start 118 71.96) (end 125.54 79.5) (width 0.2) (layer "F.Cu") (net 4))
 (segment (start 92.38 56) (end 80.979 67.401) (width 0.2) (layer "B.Cu") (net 4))
 (segment (start 92.38 56) (end 106.991 70.611) (width 0.2) (layer "B.Cu") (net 4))
 (segment (start 80.979 67.401) (end 80.979 77.021) (width 0.2) (layer "B.Cu") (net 4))
 (segment (start 80.979 77.021) (end 79.46 78.54) (width 0.2) (layer "B.Cu") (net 4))
 (segment (start 106.991 70.611) (end 116.651 70.611) (width 0.2) (layer "B.Cu") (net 4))
 (segment (start 116.651 70.611) (end 118 71.96) (width 0.2) (layer "B.Cu") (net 4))
 (segment (start 133.4125 79.5) (end 131.5275 81.385) (width 0.2) (layer "F.Cu") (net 39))
 (segment (start 138.16 80.16) (end 144 80.16) (width 0.2) (layer "F.Cu") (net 39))
 (segment (start 143.34 79.5) (end 144 80.16) (width 0.2) (layer "F.Cu") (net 39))
 (segment (start 137.5 79.5) (end 138.16 80.16) (width 0.2) (layer "F.Cu") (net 39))
 (segment (start 131.115 102.225) (end 131.115 81.385) (width 0.2) (layer "F.Cu") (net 39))
 (segment (start 133 79.5) (end 137.5 79.5) (width 0.2) (layer "F.Cu") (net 39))
 (segment (start 133.4125 79.5) (end 133.901 79.9885) (width 0.2) (layer "F.Cu") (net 39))
 (segment (start 131.5275 81.385) (end 131.115 81.385) (width 0.2) (layer "F.Cu") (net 39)))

